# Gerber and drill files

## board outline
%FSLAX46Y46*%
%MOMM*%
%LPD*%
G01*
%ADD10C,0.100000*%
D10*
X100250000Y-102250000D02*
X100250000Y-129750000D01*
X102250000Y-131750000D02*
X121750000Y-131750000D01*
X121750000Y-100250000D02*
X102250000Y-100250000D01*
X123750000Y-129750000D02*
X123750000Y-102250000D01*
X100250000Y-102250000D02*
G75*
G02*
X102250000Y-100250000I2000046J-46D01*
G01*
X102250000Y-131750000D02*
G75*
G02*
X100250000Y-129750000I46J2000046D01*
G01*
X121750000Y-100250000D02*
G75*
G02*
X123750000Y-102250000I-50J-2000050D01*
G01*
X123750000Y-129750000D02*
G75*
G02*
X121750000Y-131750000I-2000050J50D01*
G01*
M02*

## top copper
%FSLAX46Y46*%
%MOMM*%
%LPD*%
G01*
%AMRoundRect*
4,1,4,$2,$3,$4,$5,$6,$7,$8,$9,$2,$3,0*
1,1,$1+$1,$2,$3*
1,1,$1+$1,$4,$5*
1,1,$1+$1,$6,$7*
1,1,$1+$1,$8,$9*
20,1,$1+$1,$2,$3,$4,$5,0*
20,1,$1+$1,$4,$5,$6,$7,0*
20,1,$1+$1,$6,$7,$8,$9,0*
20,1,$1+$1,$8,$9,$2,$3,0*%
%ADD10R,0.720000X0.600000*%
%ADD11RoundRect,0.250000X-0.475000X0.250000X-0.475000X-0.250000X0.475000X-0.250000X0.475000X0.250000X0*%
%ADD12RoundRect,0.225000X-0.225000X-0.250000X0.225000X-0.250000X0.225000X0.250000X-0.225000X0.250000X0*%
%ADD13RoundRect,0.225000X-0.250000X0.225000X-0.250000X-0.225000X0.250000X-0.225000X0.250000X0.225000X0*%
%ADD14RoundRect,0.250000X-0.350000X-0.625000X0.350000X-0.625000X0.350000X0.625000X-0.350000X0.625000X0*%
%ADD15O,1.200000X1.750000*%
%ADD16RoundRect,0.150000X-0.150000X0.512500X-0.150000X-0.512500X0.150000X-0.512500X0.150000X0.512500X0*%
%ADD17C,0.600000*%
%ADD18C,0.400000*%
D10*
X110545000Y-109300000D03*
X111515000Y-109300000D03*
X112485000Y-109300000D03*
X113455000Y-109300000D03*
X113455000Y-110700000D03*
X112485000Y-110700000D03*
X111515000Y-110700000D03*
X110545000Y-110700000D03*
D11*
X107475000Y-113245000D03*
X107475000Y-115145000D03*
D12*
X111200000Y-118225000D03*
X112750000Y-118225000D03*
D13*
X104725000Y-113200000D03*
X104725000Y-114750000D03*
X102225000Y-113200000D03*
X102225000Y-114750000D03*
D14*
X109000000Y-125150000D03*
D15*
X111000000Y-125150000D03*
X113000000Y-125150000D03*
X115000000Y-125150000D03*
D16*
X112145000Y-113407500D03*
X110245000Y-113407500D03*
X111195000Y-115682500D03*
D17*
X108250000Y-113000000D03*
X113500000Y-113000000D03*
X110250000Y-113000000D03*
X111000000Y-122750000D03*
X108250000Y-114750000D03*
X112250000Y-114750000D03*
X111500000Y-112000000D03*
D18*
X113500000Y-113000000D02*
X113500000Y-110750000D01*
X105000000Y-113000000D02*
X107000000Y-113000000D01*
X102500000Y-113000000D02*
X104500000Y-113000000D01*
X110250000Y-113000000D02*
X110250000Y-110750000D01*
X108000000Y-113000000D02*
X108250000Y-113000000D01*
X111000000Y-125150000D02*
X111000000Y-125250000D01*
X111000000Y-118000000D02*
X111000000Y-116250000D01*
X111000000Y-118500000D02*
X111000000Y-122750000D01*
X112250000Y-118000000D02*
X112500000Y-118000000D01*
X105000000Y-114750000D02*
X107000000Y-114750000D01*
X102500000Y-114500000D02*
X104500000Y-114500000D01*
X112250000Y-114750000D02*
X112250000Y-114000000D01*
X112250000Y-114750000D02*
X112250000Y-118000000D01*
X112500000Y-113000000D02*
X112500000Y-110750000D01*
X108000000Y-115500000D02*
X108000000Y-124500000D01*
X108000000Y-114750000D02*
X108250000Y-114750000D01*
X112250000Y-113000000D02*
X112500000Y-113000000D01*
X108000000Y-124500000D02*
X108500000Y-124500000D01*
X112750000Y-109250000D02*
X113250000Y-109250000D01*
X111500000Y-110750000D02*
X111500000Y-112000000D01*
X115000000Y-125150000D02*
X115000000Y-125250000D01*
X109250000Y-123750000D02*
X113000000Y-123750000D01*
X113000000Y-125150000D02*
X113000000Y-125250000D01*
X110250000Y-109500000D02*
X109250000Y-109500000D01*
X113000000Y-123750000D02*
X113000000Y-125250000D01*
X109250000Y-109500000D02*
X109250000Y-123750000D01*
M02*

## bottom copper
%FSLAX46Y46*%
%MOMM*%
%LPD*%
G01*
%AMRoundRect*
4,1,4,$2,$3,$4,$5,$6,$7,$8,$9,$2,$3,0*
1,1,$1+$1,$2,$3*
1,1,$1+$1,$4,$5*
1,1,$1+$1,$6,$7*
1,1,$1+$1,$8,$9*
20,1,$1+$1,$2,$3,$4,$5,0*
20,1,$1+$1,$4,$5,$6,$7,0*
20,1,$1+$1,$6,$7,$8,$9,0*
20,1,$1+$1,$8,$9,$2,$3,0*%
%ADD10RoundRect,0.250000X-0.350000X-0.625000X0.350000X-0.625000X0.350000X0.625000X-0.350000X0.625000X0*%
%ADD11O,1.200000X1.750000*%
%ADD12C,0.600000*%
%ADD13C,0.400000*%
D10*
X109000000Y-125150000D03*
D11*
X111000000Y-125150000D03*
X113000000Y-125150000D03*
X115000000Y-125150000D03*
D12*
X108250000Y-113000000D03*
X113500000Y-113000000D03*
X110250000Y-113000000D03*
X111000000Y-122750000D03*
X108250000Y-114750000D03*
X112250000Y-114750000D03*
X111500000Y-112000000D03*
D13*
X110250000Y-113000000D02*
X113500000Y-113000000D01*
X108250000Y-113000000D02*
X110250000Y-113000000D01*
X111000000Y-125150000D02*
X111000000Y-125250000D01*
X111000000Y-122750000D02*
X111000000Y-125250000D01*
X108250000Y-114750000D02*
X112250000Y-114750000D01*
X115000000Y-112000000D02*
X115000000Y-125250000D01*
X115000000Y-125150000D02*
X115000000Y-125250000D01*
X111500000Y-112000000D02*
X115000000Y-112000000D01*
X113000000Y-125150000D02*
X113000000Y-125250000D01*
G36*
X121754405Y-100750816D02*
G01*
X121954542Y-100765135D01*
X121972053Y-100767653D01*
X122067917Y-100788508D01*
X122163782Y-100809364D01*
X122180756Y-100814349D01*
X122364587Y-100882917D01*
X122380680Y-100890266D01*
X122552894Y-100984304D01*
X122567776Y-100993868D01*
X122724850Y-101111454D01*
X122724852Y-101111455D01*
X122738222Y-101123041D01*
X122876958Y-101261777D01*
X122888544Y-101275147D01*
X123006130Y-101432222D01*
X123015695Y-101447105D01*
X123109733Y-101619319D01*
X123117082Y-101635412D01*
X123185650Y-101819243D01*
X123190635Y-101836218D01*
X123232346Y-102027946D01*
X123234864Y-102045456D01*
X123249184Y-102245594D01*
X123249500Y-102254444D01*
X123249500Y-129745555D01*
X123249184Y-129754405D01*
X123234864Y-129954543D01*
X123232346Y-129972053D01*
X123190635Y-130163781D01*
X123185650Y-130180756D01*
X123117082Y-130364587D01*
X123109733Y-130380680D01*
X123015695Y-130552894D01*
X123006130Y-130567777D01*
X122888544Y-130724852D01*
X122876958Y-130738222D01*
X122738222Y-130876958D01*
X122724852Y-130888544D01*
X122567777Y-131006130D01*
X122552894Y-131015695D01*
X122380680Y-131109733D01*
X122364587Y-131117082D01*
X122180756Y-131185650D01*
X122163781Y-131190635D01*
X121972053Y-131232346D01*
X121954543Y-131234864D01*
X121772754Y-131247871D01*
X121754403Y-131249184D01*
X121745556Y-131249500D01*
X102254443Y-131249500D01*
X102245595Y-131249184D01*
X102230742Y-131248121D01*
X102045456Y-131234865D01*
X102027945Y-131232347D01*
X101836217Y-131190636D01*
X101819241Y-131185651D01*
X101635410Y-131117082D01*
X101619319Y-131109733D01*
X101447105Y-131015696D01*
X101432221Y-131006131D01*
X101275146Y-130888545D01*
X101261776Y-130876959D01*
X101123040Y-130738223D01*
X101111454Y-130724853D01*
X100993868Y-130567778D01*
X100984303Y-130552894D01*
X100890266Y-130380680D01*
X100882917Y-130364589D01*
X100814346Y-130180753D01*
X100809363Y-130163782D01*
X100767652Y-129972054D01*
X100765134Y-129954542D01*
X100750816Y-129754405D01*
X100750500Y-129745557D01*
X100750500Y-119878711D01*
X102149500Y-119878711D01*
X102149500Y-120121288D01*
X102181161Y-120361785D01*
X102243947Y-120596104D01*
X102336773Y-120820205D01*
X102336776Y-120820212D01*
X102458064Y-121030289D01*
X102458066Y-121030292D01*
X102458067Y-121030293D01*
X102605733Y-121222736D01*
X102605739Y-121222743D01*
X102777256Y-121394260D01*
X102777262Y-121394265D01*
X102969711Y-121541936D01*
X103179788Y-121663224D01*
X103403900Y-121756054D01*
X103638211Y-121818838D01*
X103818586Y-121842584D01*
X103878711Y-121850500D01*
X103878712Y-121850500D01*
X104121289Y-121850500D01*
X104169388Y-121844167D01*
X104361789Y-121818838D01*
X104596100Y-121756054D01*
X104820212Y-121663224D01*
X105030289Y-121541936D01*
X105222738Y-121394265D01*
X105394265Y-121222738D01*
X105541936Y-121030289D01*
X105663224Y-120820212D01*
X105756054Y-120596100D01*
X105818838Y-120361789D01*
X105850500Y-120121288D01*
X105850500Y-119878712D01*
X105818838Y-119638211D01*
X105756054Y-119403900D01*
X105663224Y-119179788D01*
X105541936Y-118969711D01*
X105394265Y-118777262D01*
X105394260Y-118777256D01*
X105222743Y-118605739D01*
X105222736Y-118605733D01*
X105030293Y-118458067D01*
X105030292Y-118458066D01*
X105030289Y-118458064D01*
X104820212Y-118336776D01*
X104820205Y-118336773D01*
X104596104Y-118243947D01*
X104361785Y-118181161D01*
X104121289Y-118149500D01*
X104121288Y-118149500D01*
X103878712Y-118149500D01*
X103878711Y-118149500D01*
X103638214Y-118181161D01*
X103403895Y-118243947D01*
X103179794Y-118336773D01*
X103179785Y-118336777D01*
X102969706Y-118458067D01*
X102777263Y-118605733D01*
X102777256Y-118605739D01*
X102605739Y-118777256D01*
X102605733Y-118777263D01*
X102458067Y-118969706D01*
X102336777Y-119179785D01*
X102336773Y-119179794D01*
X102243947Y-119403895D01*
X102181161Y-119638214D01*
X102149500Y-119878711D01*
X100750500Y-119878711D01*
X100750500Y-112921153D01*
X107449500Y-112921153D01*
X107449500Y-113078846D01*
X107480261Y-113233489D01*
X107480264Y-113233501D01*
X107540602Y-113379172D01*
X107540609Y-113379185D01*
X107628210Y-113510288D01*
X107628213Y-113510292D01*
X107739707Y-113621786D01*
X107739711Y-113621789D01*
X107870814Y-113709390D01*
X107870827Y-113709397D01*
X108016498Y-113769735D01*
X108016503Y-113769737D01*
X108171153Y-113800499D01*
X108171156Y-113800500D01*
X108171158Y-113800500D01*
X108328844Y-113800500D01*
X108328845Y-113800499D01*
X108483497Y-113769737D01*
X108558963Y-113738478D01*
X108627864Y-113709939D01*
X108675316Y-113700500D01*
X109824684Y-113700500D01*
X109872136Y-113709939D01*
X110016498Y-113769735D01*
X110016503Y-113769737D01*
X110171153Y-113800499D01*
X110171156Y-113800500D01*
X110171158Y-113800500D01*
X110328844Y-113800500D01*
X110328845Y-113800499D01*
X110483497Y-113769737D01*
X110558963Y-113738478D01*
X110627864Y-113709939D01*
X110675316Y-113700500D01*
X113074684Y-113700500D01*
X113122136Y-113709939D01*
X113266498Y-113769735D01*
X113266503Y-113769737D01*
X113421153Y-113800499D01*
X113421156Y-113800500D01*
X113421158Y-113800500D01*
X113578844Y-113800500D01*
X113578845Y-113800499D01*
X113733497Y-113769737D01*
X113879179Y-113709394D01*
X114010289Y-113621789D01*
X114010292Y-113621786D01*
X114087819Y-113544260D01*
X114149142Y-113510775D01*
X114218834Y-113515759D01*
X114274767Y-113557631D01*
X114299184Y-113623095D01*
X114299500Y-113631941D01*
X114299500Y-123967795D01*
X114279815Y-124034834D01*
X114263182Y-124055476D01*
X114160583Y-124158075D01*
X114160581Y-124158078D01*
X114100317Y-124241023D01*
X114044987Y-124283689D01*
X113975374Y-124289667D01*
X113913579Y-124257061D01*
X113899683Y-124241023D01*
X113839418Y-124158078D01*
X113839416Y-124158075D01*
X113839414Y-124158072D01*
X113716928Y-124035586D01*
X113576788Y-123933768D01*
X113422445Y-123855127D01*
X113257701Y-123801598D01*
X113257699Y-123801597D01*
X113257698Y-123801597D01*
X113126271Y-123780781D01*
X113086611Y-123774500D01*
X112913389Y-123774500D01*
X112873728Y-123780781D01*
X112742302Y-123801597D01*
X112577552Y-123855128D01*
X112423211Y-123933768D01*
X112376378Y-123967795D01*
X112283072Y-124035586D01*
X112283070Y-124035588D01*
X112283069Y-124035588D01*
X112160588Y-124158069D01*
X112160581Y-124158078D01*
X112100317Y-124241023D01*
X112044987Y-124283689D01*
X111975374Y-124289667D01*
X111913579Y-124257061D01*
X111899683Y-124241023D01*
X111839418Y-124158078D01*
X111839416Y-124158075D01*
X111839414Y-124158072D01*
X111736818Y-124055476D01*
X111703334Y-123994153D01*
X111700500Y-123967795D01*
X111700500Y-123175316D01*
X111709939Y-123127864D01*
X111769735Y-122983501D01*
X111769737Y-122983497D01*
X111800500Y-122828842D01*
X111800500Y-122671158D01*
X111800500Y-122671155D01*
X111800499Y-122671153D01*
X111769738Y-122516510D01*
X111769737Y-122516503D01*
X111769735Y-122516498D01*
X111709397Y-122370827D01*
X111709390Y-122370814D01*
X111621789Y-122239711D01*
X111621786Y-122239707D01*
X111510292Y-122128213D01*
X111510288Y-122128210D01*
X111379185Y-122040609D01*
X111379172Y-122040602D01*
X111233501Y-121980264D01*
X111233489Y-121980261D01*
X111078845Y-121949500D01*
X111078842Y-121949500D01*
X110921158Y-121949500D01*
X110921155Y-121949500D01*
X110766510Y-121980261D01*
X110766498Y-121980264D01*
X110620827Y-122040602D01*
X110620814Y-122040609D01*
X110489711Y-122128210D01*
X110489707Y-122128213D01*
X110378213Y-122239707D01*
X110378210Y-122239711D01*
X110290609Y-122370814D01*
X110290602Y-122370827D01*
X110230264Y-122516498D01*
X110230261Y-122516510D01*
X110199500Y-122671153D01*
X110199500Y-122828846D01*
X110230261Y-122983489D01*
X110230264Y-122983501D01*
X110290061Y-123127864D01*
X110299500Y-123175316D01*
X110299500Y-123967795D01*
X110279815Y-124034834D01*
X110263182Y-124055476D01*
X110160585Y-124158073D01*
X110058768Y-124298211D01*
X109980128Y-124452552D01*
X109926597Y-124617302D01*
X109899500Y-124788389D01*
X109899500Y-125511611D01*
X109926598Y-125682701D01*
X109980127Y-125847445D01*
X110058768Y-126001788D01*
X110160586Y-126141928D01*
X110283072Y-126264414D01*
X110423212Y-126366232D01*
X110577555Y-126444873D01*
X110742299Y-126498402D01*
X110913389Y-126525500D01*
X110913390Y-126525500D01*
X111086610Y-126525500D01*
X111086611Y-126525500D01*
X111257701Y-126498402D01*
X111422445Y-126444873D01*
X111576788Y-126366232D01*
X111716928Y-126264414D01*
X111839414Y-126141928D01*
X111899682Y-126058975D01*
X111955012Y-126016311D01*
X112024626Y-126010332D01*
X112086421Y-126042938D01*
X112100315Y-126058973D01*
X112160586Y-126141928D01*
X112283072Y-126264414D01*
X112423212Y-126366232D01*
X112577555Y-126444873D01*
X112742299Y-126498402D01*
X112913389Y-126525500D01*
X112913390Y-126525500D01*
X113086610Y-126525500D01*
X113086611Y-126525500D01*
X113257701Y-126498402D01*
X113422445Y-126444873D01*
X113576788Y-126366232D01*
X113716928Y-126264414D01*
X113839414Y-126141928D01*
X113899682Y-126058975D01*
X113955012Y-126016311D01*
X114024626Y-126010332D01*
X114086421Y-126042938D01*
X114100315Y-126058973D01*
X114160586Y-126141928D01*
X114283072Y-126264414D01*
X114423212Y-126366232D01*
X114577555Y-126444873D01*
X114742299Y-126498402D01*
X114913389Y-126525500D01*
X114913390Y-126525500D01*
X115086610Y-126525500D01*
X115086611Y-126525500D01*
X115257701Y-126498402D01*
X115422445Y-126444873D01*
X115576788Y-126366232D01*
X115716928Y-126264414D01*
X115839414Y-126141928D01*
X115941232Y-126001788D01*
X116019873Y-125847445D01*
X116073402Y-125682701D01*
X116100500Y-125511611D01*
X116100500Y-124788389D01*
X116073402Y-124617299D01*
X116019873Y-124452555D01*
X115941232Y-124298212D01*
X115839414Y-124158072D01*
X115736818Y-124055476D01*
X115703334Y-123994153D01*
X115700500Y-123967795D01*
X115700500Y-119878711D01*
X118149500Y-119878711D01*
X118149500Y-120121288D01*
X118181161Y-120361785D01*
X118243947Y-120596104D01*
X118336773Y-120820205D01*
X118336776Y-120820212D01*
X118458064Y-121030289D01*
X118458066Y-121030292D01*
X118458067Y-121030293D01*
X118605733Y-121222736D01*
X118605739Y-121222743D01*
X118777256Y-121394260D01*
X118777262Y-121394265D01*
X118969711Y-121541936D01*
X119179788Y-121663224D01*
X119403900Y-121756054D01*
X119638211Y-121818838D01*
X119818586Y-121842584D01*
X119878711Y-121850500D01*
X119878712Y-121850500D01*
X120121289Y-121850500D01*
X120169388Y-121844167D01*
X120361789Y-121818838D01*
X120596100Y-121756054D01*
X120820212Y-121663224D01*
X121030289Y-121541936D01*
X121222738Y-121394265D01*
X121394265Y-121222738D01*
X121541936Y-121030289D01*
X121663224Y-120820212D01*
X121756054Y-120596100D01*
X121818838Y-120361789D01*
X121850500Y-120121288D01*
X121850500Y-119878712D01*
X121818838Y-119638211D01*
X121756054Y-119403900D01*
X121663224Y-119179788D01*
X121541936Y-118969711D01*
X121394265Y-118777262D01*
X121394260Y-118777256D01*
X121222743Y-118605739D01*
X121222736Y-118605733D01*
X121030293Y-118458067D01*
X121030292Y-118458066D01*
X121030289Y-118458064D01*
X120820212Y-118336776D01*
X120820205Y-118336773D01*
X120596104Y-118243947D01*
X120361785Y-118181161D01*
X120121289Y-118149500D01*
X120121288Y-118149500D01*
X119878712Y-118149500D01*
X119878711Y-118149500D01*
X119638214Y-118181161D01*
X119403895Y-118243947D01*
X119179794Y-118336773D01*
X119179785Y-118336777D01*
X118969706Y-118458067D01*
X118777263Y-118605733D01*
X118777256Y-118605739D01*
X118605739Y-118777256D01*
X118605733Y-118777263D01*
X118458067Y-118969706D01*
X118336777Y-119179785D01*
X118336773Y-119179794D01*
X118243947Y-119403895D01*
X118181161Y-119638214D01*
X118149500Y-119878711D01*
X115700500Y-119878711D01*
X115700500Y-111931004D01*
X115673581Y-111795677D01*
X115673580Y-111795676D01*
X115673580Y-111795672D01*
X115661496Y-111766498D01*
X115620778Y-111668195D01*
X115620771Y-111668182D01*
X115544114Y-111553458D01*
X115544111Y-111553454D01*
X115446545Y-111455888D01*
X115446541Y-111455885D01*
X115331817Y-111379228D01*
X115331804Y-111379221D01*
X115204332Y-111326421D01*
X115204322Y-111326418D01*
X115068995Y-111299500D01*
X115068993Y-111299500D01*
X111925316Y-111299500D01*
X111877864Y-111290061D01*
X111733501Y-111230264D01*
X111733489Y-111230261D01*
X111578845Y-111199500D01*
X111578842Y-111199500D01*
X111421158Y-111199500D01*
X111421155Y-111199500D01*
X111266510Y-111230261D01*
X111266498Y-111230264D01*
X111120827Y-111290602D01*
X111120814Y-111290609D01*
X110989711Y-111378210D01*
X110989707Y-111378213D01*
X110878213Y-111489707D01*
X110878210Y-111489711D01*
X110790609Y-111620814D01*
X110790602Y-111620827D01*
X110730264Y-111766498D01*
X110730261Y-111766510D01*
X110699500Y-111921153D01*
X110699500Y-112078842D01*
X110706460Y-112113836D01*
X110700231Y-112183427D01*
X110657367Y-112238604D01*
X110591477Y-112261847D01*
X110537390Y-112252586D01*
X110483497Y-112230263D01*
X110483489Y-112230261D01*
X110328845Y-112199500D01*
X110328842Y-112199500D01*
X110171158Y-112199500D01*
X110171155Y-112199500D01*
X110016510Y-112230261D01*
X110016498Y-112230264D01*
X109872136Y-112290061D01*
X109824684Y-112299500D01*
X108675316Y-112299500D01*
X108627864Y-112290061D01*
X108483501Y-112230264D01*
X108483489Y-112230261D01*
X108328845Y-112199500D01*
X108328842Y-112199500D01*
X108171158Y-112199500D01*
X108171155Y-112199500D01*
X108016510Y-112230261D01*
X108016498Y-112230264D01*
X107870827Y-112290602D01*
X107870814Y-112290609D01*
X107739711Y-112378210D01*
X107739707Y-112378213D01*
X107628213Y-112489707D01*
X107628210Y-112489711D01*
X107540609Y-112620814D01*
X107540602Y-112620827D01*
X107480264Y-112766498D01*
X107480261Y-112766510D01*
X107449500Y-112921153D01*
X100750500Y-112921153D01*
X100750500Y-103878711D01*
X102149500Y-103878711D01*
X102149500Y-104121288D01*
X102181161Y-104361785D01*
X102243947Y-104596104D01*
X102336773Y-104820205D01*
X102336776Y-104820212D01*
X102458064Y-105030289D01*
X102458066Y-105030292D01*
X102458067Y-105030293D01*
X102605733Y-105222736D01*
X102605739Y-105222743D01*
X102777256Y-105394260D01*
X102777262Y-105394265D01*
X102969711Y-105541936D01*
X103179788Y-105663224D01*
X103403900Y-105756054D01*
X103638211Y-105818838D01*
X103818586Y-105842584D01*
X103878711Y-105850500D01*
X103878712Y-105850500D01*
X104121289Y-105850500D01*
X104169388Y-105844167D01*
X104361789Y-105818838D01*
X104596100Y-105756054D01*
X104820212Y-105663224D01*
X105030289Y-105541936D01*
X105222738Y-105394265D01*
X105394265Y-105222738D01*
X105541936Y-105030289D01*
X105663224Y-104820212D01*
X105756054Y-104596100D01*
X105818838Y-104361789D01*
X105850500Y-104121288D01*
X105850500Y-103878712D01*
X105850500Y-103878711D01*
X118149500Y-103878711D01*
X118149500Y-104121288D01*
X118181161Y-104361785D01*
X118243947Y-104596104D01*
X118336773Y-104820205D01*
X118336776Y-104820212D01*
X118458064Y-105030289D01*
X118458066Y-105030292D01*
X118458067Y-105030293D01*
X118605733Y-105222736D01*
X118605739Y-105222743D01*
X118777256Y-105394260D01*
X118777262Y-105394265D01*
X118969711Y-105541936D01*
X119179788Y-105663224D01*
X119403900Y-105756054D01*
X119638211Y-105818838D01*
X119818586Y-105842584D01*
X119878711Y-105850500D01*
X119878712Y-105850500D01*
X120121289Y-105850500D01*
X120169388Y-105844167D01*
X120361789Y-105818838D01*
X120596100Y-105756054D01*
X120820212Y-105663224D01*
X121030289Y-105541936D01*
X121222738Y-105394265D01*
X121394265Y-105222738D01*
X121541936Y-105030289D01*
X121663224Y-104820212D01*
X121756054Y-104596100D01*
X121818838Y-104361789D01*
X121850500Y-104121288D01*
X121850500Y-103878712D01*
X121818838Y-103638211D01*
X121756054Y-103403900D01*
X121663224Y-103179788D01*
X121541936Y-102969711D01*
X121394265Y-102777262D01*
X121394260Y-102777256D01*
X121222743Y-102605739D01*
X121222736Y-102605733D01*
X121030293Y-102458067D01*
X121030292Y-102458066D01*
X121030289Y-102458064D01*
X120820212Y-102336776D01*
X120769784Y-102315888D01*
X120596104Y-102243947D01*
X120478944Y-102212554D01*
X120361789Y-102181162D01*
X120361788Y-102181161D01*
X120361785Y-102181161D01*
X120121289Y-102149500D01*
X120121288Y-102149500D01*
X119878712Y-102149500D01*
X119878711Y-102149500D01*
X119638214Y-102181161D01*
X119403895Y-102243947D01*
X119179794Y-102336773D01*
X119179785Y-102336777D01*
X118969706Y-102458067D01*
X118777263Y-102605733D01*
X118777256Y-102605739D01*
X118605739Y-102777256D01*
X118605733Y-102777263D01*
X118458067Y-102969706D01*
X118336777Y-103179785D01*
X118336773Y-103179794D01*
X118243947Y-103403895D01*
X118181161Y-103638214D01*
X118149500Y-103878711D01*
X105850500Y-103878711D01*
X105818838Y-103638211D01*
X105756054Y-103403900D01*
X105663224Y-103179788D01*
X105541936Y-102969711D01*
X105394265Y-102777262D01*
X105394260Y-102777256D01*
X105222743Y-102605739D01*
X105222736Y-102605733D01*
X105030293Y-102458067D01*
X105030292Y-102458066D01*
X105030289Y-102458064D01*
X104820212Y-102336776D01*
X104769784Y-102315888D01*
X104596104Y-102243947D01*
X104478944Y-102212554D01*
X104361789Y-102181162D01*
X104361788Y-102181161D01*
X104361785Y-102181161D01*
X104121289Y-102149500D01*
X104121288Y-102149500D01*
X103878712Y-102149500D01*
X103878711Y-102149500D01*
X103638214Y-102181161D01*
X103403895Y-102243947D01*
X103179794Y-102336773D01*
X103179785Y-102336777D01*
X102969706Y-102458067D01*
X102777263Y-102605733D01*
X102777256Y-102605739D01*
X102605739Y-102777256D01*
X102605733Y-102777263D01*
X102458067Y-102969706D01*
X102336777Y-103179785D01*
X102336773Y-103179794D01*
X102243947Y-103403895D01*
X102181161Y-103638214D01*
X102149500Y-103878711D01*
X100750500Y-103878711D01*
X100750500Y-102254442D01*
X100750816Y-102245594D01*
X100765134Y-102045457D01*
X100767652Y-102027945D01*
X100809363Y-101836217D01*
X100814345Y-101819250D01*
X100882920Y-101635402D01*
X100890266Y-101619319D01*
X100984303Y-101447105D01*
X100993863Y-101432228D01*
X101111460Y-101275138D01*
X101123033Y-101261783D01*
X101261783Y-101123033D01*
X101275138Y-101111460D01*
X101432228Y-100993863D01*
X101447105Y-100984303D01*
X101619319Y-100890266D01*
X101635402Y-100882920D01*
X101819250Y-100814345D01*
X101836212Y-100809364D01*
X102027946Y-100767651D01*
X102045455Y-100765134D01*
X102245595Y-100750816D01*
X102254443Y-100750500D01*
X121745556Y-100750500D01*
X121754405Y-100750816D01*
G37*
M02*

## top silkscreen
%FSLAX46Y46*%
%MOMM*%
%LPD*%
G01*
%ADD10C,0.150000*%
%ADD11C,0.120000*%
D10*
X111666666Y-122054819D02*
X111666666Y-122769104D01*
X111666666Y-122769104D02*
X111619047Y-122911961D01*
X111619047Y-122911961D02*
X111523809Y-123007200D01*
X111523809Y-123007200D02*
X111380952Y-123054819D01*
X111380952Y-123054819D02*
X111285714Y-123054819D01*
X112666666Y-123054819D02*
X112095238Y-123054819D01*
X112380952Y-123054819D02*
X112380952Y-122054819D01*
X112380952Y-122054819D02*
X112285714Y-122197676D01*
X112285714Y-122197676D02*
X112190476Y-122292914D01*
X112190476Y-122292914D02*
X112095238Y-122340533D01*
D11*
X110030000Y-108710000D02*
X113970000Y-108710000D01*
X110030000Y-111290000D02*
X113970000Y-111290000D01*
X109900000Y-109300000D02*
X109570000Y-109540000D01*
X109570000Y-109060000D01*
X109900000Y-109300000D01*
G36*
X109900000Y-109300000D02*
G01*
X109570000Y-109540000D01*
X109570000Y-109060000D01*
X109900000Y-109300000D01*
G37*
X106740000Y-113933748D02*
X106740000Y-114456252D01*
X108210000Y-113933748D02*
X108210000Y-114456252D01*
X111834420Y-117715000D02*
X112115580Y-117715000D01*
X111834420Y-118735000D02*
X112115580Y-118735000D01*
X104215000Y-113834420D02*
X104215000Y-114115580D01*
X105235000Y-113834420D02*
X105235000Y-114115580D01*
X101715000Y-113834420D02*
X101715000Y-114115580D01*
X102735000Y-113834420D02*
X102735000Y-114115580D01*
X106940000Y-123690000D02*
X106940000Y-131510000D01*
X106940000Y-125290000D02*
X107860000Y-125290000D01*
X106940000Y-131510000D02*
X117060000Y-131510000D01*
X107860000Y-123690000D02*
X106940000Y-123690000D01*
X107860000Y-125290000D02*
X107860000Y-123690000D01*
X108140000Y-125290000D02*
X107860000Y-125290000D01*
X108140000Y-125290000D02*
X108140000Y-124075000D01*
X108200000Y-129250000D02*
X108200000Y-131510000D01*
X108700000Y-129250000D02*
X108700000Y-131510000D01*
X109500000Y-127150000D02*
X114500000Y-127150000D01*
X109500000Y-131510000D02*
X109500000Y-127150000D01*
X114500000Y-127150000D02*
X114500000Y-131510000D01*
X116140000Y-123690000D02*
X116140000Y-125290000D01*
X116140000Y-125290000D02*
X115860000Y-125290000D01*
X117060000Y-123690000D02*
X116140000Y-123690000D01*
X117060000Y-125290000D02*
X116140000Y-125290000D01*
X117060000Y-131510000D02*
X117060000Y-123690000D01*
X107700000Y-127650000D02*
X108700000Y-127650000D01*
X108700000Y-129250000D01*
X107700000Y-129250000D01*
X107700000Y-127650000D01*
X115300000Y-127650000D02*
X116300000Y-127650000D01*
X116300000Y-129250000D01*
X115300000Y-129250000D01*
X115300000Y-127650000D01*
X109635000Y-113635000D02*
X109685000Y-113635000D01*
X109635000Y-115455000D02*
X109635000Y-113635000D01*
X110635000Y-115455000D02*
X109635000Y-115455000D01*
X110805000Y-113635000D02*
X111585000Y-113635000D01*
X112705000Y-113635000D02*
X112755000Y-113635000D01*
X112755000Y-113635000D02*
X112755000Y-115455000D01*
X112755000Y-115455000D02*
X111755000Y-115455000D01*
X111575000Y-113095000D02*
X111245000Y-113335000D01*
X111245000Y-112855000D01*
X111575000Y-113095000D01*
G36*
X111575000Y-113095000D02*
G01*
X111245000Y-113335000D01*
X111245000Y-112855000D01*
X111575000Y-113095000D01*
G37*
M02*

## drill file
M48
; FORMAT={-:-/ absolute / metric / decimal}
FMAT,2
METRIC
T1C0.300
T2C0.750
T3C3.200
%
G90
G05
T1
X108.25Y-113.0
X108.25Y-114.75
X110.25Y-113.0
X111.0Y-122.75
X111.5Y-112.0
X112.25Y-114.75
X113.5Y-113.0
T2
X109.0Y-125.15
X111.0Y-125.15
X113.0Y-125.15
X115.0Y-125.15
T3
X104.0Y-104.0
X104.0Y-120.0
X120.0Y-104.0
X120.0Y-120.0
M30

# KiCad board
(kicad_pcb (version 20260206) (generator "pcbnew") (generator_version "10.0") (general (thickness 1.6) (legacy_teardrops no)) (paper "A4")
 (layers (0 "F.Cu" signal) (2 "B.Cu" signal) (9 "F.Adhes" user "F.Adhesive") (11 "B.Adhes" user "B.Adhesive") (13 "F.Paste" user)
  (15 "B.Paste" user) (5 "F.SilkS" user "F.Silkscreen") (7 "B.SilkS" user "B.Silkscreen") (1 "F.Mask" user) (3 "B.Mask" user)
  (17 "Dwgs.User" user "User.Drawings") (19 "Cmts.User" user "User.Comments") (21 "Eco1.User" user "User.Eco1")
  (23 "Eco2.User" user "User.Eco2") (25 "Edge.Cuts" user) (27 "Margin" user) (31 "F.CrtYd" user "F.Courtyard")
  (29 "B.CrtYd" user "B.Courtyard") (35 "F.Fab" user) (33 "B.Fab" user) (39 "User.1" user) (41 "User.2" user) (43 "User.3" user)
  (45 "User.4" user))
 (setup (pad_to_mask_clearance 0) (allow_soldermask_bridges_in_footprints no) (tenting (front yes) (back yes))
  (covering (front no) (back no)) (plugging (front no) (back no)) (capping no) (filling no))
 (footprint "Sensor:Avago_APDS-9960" (layer "F.Cu") (at 112 110)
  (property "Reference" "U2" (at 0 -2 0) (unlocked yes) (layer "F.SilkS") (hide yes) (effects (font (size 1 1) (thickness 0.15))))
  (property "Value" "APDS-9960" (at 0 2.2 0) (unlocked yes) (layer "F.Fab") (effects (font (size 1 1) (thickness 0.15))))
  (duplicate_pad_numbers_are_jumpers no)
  (fp_line (start -1.97 -1.29) (end 1.97 -1.29) (stroke (width 0.12) (type solid)) (layer "F.SilkS"))
  (fp_line (start -1.97 1.29) (end 1.97 1.29) (stroke (width 0.12) (type solid)) (layer "F.SilkS"))
  (fp_poly
   (pts (xy -2.1 -0.7) (xy -2.43 -0.46) (xy -2.43 -0.94) (xy -2.1 -0.7)) (stroke (width 0.12) (type solid)) (fill yes) (layer "F.SilkS"))
  (pad "1" smd rect (at -1.455 -0.7) (size 0.72 0.6) (layers "F.Cu" "F.Mask" "F.Paste") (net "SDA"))
  (pad "2" smd rect (at -0.485 -0.7) (size 0.72 0.6) (layers "F.Cu" "F.Mask" "F.Paste") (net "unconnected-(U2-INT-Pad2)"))
  (pad "3" smd rect (at 0.485 -0.7) (size 0.72 0.6) (layers "F.Cu" "F.Mask" "F.Paste") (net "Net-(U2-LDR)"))
  (pad "4" smd rect (at 1.455 -0.7) (size 0.72 0.6) (layers "F.Cu" "F.Mask" "F.Paste") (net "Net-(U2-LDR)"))
  (pad "5" smd rect (at 1.455 0.7) (size 0.72 0.6) (layers "F.Cu" "F.Mask" "F.Paste") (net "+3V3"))
  (pad "6" smd rect (at 0.485 0.7) (size 0.72 0.6) (layers "F.Cu" "F.Mask" "F.Paste") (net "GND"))
  (pad "7" smd rect (at -0.485 0.7) (size 0.72 0.6) (layers "F.Cu" "F.Mask" "F.Paste") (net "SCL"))
  (pad "8" smd rect (at -1.455 0.7) (size 0.72 0.6) (layers "F.Cu" "F.Mask" "F.Paste") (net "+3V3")))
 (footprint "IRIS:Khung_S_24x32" (layer "F.Cu") (at 100 132)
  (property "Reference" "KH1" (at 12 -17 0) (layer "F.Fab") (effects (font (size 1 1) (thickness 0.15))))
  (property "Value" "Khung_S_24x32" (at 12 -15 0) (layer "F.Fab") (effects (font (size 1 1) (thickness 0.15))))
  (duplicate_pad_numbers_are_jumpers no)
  (fp_line (start 0.25 -29.75) (end 0.25 -2.25) (stroke (width 0.1) (type solid)) (layer "Edge.Cuts"))
  (fp_line (start 2.25 -0.25) (end 21.75 -0.25) (stroke (width 0.1) (type solid)) (layer "Edge.Cuts"))
  (fp_line (start 21.75 -31.75) (end 2.25 -31.75) (stroke (width 0.1) (type solid)) (layer "Edge.Cuts"))
  (fp_line (start 23.75 -2.25) (end 23.75 -29.75) (stroke (width 0.1) (type solid)) (layer "Edge.Cuts"))
  (fp_arc (start 0.25 -29.75) (mid 0.8358 -31.1642) (end 2.25 -31.75) (stroke (width 0.1) (type solid)) (layer "Edge.Cuts"))
  (fp_arc (start 2.25 -0.25) (mid 0.8358 -0.8358) (end 0.25 -2.25) (stroke (width 0.1) (type solid)) (layer "Edge.Cuts"))
  (fp_arc (start 21.75 -31.75) (mid 23.164199 -31.164199) (end 23.75 -29.75) (stroke (width 0.1) (type solid)) (layer "Edge.Cuts"))
  (fp_arc (start 23.75 -2.25) (mid 23.164199 -0.835801) (end 21.75 -0.25) (stroke (width 0.1) (type solid)) (layer "Edge.Cuts"))
  (pad "" np_thru_hole circle (at 4 -28) (size 3.2 3.2) (drill 3.2) (layers "*.Cu" "*.Mask"))
  (pad "" np_thru_hole circle (at 4 -12) (size 3.2 3.2) (drill 3.2) (layers "*.Cu" "*.Mask"))
  (pad "" np_thru_hole circle (at 20 -28) (size 3.2 3.2) (drill 3.2) (layers "*.Cu" "*.Mask"))
  (pad "" np_thru_hole circle (at 20 -12) (size 3.2 3.2) (drill 3.2) (layers "*.Cu" "*.Mask")))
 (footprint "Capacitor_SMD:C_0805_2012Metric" (layer "F.Cu") (at 107.475 114.195 -90)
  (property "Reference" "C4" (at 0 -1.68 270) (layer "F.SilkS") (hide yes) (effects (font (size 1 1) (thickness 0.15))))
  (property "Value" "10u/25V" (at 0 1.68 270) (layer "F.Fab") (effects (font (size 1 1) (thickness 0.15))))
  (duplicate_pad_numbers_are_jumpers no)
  (fp_line (start -0.261252 0.735) (end 0.261252 0.735) (stroke (width 0.12) (type solid)) (layer "F.SilkS"))
  (fp_line (start -0.261252 -0.735) (end 0.261252 -0.735) (stroke (width 0.12) (type solid)) (layer "F.SilkS"))
  (pad "1" smd roundrect (at -0.95 0 270) (size 1 1.45) (layers "F.Cu" "F.Mask" "F.Paste") (roundrect_rratio 0.25) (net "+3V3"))
  (pad "2" smd roundrect (at 0.95 0 270) (size 1 1.45) (layers "F.Cu" "F.Mask" "F.Paste") (roundrect_rratio 0.25) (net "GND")))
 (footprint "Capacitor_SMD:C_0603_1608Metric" (layer "F.Cu") (at 111.975 118.225)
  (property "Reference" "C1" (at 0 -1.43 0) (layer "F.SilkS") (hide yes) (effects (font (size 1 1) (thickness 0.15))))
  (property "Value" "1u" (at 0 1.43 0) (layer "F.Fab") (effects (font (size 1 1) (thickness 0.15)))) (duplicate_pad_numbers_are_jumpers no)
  (fp_line (start -0.14058 -0.51) (end 0.14058 -0.51) (stroke (width 0.12) (type solid)) (layer "F.SilkS"))
  (fp_line (start -0.14058 0.51) (end 0.14058 0.51) (stroke (width 0.12) (type solid)) (layer "F.SilkS"))
  (pad "1" smd roundrect (at -0.775 0) (size 0.9 0.95) (layers "F.Cu" "F.Mask" "F.Paste") (roundrect_rratio 0.25) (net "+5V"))
  (pad "2" smd roundrect (at 0.775 0) (size 0.9 0.95) (layers "F.Cu" "F.Mask" "F.Paste") (roundrect_rratio 0.25) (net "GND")))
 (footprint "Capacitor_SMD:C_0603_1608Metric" (layer "F.Cu") (at 104.725 113.975 -90)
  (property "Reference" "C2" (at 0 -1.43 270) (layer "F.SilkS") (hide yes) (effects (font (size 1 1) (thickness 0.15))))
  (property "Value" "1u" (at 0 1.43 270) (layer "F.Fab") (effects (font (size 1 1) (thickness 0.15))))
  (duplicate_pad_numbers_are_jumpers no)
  (fp_line (start -0.14058 0.51) (end 0.14058 0.51) (stroke (width 0.12) (type solid)) (layer "F.SilkS"))
  (fp_line (start -0.14058 -0.51) (end 0.14058 -0.51) (stroke (width 0.12) (type solid)) (layer "F.SilkS"))
  (pad "1" smd roundrect (at -0.775 0 270) (size 0.9 0.95) (layers "F.Cu" "F.Mask" "F.Paste") (roundrect_rratio 0.25) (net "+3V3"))
  (pad "2" smd roundrect (at 0.775 0 270) (size 0.9 0.95) (layers "F.Cu" "F.Mask" "F.Paste") (roundrect_rratio 0.25) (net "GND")))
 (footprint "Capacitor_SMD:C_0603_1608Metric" (layer "F.Cu") (at 102.225 113.975 -90)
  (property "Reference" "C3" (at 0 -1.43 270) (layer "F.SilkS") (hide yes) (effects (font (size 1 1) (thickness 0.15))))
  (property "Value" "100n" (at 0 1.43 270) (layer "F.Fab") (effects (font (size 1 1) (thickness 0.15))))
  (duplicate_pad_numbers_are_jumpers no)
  (fp_line (start -0.14058 0.51) (end 0.14058 0.51) (stroke (width 0.12) (type solid)) (layer "F.SilkS"))
  (fp_line (start -0.14058 -0.51) (end 0.14058 -0.51) (stroke (width 0.12) (type solid)) (layer "F.SilkS"))
  (pad "1" smd roundrect (at -0.775 0 270) (size 0.9 0.95) (layers "F.Cu" "F.Mask" "F.Paste") (roundrect_rratio 0.25) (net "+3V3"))
  (pad "2" smd roundrect (at 0.775 0 270) (size 0.9 0.95) (layers "F.Cu" "F.Mask" "F.Paste") (roundrect_rratio 0.25) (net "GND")))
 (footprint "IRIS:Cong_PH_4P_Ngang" (layer "F.Cu") (at 109 125.15)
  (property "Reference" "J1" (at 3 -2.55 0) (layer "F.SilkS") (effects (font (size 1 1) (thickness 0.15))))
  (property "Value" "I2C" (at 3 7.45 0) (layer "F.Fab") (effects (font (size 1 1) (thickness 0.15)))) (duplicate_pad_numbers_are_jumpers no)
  (fp_line (start -2.06 -1.46) (end -2.06 6.36) (stroke (width 0.12) (type solid)) (layer "F.SilkS"))
  (fp_line (start -2.06 0.14) (end -1.14 0.14) (stroke (width 0.12) (type solid)) (layer "F.SilkS"))
  (fp_line (start -2.06 6.36) (end 8.06 6.36) (stroke (width 0.12) (type solid)) (layer "F.SilkS"))
  (fp_line (start -1.14 -1.46) (end -2.06 -1.46) (stroke (width 0.12) (type solid)) (layer "F.SilkS"))
  (fp_line (start -1.14 0.14) (end -1.14 -1.46) (stroke (width 0.12) (type solid)) (layer "F.SilkS"))
  (fp_line (start -0.86 0.14) (end -1.14 0.14) (stroke (width 0.12) (type solid)) (layer "F.SilkS"))
  (fp_line (start -0.86 0.14) (end -0.86 -1.075) (stroke (width 0.12) (type solid)) (layer "F.SilkS"))
  (fp_line (start -0.8 4.1) (end -0.8 6.36) (stroke (width 0.12) (type solid)) (layer "F.SilkS"))
  (fp_line (start -0.3 4.1) (end -0.3 6.36) (stroke (width 0.12) (type solid)) (layer "F.SilkS"))
  (fp_line (start 0.5 2) (end 5.5 2) (stroke (width 0.12) (type solid)) (layer "F.SilkS"))
  (fp_line (start 0.5 6.36) (end 0.5 2) (stroke (width 0.12) (type solid)) (layer "F.SilkS"))
  (fp_line (start 5.5 2) (end 5.5 6.36) (stroke (width 0.12) (type solid)) (layer "F.SilkS"))
  (fp_line (start 7.14 -1.46) (end 7.14 0.14) (stroke (width 0.12) (type solid)) (layer "F.SilkS"))
  (fp_line (start 7.14 0.14) (end 6.86 0.14) (stroke (width 0.12) (type solid)) (layer "F.SilkS"))
  (fp_line (start 8.06 -1.46) (end 7.14 -1.46) (stroke (width 0.12) (type solid)) (layer "F.SilkS"))
  (fp_line (start 8.06 0.14) (end 7.14 0.14) (stroke (width 0.12) (type solid)) (layer "F.SilkS"))
  (fp_line (start 8.06 6.36) (end 8.06 -1.46) (stroke (width 0.12) (type solid)) (layer "F.SilkS"))
  (fp_rect (start -1.3 2.5) (end -0.3 4.1) (stroke (width 0.12) (type solid)) (fill no) (layer "F.SilkS"))
  (fp_rect (start 6.3 2.5) (end 7.3 4.1) (stroke (width 0.12) (type solid)) (fill no) (layer "F.SilkS"))
  (pad "1" thru_hole roundrect (at 0 0) (size 1.2 1.75) (drill 0.75) (layers "*.Cu" "*.Mask") (remove_unused_layers no)
   (roundrect_rratio 0.208333) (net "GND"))
  (pad "2" thru_hole oval (at 2 0) (size 1.2 1.75) (drill 0.75) (layers "*.Cu" "*.Mask") (remove_unused_layers no) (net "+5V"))
  (pad "3" thru_hole oval (at 4 0) (size 1.2 1.75) (drill 0.75) (layers "*.Cu" "*.Mask") (remove_unused_layers no) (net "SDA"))
  (pad "4" thru_hole oval (at 6 0) (size 1.2 1.75) (drill 0.75) (layers "*.Cu" "*.Mask") (remove_unused_layers no) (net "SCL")))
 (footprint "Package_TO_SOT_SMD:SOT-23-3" (layer "F.Cu") (at 111.195 114.545 -90)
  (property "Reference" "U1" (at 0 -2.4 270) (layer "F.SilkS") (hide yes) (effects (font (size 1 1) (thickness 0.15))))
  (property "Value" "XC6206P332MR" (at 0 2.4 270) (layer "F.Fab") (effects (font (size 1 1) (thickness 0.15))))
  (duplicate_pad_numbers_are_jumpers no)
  (fp_line (start -0.91 1.56) (end -0.91 1.51) (stroke (width 0.12) (type solid)) (layer "F.SilkS"))
  (fp_line (start 0.91 1.56) (end -0.91 1.56) (stroke (width 0.12) (type solid)) (layer "F.SilkS"))
  (fp_line (start 0.91 0.56) (end 0.91 1.56) (stroke (width 0.12) (type solid)) (layer "F.SilkS"))
  (fp_line (start -0.91 0.39) (end -0.91 -0.39) (stroke (width 0.12) (type solid)) (layer "F.SilkS"))
  (fp_line (start -0.91 -1.51) (end -0.91 -1.56) (stroke (width 0.12) (type solid)) (layer "F.SilkS"))
  (fp_line (start -0.91 -1.56) (end 0.91 -1.56) (stroke (width 0.12) (type solid)) (layer "F.SilkS"))
  (fp_line (start 0.91 -1.56) (end 0.91 -0.56) (stroke (width 0.12) (type solid)) (layer "F.SilkS"))
  (fp_poly (pts (xy -1.45 -0.38) (xy -1.21 -0.05) (xy -1.69 -0.05)) (stroke (width 0.12) (type solid)) (fill yes) (layer "F.SilkS"))
  (pad "1" smd roundrect (at -1.1375 -0.95 270) (size 1.325 0.6) (layers "F.Cu" "F.Mask" "F.Paste") (roundrect_rratio 0.25) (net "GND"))
  (pad "2" smd roundrect (at -1.1375 0.95 270) (size 1.325 0.6) (layers "F.Cu" "F.Mask" "F.Paste") (roundrect_rratio 0.25) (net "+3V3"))
  (pad "3" smd roundrect (at 1.1375 0 270) (size 1.325 0.6) (layers "F.Cu" "F.Mask" "F.Paste") (roundrect_rratio 0.25) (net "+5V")))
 (segment (start 113.5 113) (end 113.5 110.75) (width 0.4) (layer "F.Cu") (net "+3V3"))
 (segment (start 105 113) (end 107 113) (width 0.4) (layer "F.Cu") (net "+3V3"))
 (segment (start 102.5 113) (end 104.5 113) (width 0.4) (layer "F.Cu") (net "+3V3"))
 (segment (start 110.25 113) (end 110.25 110.75) (width 0.4) (layer "F.Cu") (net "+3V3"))
 (segment (start 108 113) (end 108.25 113) (width 0.4) (layer "F.Cu") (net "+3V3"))
 (via (at 108.25 113) (size 0.6) (drill 0.3) (layers "F.Cu" "B.Cu") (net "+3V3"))
 (via (at 113.5 113) (size 0.6) (drill 0.3) (layers "F.Cu" "B.Cu") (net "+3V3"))
 (via (at 110.25 113) (size 0.6) (drill 0.3) (layers "F.Cu" "B.Cu") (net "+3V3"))
 (segment (start 110.25 113) (end 113.5 113) (width 0.4) (layer "B.Cu") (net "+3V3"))
 (segment (start 108.25 113) (end 110.25 113) (width 0.4) (layer "B.Cu") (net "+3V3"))
 (segment (start 111 125.15) (end 111 125.25) (width 0.4) (layer "F.Cu") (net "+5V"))
 (segment (start 111 118) (end 111 116.25) (width 0.4) (layer "F.Cu") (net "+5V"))
 (segment (start 111 118.5) (end 111 122.75) (width 0.4) (layer "F.Cu") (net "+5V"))
 (via (at 111 122.75) (size 0.6) (drill 0.3) (layers "F.Cu" "B.Cu") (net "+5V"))
 (segment (start 111 125.15) (end 111 125.25) (width 0.4) (layer "B.Cu") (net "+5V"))
 (segment (start 111 122.75) (end 111 125.25) (width 0.4) (layer "B.Cu") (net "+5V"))
 (segment (start 112.25 118) (end 112.5 118) (width 0.4) (layer "F.Cu") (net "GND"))
 (segment (start 105 114.75) (end 107 114.75) (width 0.4) (layer "F.Cu") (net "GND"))
 (segment (start 102.5 114.5) (end 104.5 114.5) (width 0.4) (layer "F.Cu") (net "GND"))
 (segment (start 112.25 114.75) (end 112.25 114) (width 0.4) (layer "F.Cu") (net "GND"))
 (segment (start 112.25 114.75) (end 112.25 118) (width 0.4) (layer "F.Cu") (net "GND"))
 (segment (start 112.5 113) (end 112.5 110.75) (width 0.4) (layer "F.Cu") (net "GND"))
 (segment (start 108 115.5) (end 108 124.5) (width 0.4) (layer "F.Cu") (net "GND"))
 (segment (start 108 114.75) (end 108.25 114.75) (width 0.4) (layer "F.Cu") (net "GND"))
 (segment (start 112.25 113) (end 112.5 113) (width 0.4) (layer "F.Cu") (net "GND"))
 (segment (start 108 124.5) (end 108.5 124.5) (width 0.4) (layer "F.Cu") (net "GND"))
 (via (at 108.25 114.75) (size 0.6) (drill 0.3) (layers "F.Cu" "B.Cu") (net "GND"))
 (via (at 112.25 114.75) (size 0.6) (drill 0.3) (layers "F.Cu" "B.Cu") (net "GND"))
 (segment (start 108.25 114.75) (end 112.25 114.75) (width 0.4) (layer "B.Cu") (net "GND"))
 (segment (start 112.75 109.25) (end 113.25 109.25) (width 0.4) (layer "F.Cu") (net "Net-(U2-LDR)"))
 (segment (start 111.5 110.75) (end 111.5 112) (width 0.4) (layer "F.Cu") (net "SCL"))
 (segment (start 115 125.15) (end 115 125.25) (width 0.4) (layer "F.Cu") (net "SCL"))
 (via (at 111.5 112) (size 0.6) (drill 0.3) (layers "F.Cu" "B.Cu") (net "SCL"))
 (segment (start 115 112) (end 115 125.25) (width 0.4) (layer "B.Cu") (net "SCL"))
 (segment (start 115 125.15) (end 115 125.25) (width 0.4) (layer "B.Cu") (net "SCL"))
 (segment (start 111.5 112) (end 115 112) (width 0.4) (layer "B.Cu") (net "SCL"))
 (segment (start 109.25 123.75) (end 113 123.75) (width 0.4) (layer "F.Cu") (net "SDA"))
 (segment (start 113 125.15) (end 113 125.25) (width 0.4) (layer "F.Cu") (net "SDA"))
 (segment (start 110.25 109.5) (end 109.25 109.5) (width 0.4) (layer "F.Cu") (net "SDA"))
 (segment (start 113 123.75) (end 113 125.25) (width 0.4) (layer "F.Cu") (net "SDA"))
 (segment (start 109.25 109.5) (end 109.25 123.75) (width 0.4) (layer "F.Cu") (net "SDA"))
 (segment (start 113 125.15) (end 113 125.25) (width 0.4) (layer "B.Cu") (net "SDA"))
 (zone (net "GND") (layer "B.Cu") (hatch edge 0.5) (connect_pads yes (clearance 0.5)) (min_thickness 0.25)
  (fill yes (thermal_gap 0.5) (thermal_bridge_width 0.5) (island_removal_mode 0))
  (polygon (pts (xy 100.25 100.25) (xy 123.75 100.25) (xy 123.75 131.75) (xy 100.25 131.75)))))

